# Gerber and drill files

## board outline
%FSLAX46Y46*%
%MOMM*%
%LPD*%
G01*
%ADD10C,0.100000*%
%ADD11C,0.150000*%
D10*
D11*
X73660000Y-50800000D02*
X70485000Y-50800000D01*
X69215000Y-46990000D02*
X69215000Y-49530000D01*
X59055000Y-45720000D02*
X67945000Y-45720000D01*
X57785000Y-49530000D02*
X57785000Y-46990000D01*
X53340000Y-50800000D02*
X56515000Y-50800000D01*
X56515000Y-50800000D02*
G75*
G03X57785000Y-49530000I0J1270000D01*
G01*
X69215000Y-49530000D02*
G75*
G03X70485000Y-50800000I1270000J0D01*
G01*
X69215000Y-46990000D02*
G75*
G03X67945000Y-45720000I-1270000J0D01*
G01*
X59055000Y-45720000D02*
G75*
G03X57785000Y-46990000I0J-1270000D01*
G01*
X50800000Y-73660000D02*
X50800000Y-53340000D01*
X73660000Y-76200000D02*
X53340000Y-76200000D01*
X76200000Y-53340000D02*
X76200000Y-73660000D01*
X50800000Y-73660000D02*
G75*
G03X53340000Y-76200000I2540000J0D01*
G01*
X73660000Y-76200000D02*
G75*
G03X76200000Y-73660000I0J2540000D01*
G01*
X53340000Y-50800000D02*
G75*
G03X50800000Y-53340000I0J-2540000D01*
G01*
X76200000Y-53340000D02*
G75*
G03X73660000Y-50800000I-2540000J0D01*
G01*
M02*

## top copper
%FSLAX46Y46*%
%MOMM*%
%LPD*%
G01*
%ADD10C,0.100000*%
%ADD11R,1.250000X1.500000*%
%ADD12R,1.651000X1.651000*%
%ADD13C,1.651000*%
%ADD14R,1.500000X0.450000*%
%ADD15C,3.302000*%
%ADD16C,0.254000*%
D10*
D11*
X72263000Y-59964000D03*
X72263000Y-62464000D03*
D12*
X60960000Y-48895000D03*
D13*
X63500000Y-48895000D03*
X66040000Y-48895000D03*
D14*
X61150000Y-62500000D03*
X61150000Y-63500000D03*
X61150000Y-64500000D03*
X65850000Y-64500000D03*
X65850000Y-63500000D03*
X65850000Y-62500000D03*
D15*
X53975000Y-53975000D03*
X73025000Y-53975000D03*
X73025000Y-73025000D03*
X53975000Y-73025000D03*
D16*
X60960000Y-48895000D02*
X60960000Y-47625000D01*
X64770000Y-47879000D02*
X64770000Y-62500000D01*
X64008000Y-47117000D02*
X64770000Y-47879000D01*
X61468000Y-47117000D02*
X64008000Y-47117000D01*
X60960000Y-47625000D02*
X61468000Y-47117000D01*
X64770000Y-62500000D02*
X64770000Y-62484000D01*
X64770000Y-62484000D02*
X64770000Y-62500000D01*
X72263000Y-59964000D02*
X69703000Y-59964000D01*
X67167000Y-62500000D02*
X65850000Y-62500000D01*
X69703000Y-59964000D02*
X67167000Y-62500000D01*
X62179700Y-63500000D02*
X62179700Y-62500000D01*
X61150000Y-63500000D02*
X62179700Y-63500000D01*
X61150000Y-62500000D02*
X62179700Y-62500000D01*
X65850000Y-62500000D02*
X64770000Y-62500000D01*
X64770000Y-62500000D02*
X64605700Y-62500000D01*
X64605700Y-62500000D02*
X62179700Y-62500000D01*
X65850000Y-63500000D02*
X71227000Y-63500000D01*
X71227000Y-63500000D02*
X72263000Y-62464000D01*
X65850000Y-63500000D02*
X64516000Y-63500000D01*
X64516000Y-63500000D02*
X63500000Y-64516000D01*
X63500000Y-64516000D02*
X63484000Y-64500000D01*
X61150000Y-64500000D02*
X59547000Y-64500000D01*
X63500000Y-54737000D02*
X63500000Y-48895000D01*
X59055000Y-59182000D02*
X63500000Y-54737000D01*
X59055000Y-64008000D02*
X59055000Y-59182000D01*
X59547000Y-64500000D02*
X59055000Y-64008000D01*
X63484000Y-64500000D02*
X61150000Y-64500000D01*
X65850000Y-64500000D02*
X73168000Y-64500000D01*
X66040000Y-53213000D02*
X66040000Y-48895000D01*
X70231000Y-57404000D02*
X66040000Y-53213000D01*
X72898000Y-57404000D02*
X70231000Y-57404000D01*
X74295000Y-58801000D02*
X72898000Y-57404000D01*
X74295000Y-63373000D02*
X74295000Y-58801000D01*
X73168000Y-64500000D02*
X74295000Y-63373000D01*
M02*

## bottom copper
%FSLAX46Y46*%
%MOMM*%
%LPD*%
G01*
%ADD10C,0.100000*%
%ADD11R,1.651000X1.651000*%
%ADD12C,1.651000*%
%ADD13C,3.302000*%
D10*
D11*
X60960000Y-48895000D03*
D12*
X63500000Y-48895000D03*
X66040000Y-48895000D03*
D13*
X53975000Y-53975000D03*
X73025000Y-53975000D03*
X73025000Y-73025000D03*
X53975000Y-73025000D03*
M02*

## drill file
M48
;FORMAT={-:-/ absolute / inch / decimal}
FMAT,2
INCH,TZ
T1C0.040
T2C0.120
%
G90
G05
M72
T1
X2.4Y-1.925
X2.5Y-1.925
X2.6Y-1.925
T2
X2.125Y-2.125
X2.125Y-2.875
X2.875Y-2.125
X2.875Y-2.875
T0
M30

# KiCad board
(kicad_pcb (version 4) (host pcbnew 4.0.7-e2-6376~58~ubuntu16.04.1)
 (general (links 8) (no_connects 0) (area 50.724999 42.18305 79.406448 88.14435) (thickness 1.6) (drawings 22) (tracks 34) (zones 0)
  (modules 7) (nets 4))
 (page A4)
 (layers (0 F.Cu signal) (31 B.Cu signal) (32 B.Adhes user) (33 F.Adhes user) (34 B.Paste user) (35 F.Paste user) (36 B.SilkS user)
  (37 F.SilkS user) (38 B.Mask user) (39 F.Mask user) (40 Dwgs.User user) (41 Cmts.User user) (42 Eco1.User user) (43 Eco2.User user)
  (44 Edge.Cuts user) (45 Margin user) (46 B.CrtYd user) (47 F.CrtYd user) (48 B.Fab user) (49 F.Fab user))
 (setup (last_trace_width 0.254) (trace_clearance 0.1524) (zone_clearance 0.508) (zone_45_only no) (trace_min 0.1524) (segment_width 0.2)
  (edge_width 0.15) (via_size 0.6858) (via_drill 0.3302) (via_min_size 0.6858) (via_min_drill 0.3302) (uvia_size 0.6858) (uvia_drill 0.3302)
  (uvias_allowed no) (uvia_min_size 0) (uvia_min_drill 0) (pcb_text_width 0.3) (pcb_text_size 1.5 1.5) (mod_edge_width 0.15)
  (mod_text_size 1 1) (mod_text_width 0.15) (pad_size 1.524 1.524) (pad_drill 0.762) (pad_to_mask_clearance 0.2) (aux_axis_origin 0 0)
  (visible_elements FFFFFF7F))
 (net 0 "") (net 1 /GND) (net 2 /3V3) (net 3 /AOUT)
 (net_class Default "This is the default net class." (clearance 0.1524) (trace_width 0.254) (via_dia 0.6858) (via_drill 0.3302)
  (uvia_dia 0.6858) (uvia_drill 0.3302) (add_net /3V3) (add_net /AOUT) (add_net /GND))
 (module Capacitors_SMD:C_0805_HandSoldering (layer F.Cu) (at 72.263 61.214 270)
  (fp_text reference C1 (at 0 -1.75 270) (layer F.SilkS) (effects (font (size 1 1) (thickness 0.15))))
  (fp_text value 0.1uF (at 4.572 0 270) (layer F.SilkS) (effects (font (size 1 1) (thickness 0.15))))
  (pad 1 smd rect (at -1.25 0 270) (size 1.5 1.25) (layers F.Cu F.Paste F.Mask) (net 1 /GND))
  (pad 2 smd rect (at 1.25 0 270) (size 1.5 1.25) (layers F.Cu F.Paste F.Mask) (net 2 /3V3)))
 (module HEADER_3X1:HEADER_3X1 (layer F.Cu) (at 63.5 48.895)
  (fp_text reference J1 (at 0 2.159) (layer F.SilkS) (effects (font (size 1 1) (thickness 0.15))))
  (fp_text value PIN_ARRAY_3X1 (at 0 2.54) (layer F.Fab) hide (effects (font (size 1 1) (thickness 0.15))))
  (pad 1 thru_hole rect (at -2.54 0) (size 1.651 1.651) (drill 1.016) (layers *.Cu *.Mask) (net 1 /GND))
  (pad 2 thru_hole circle (at 0 0) (size 1.651 1.651) (drill 1.016) (layers *.Cu *.Mask) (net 2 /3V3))
  (pad 3 thru_hole circle (at 2.54 0) (size 1.651 1.651) (drill 1.016) (layers *.Cu *.Mask) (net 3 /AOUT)))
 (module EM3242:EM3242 (layer F.Cu) (at 63.5 63.5)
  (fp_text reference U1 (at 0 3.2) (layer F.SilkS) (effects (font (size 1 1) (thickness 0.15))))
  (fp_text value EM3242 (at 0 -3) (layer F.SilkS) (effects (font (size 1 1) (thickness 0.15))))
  (pad 1 smd rect (at -2.35 -1) (size 1.5 0.45) (layers F.Cu F.Paste F.Mask) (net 1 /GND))
  (pad 2 smd rect (at -2.35 0) (size 1.5 0.45) (layers F.Cu F.Paste F.Mask) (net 1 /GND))
  (pad 3 smd rect (at -2.35 1) (size 1.5 0.45) (layers F.Cu F.Paste F.Mask) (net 2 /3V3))
  (pad 4 smd rect (at 2.35 1) (size 1.5 0.45) (layers F.Cu F.Paste F.Mask) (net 3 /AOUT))
  (pad 5 smd rect (at 2.35 0) (size 1.5 0.45) (layers F.Cu F.Paste F.Mask) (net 2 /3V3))
  (pad 6 smd rect (at 2.35 -1) (size 1.5 0.45) (layers F.Cu F.Paste F.Mask) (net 1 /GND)))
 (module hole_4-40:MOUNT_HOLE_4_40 (layer F.Cu) (at 53.34 53.34)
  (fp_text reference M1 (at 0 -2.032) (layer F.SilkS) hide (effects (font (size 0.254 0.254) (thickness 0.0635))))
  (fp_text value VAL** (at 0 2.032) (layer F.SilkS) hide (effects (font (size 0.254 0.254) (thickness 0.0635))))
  (pad "" thru_hole circle (at 0.635 0.635) (size 3.302 3.302) (drill 3.048) (layers *.Cu *.SilkS *.Mask)))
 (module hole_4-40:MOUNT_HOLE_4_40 (layer F.Cu) (at 75.057 44.577)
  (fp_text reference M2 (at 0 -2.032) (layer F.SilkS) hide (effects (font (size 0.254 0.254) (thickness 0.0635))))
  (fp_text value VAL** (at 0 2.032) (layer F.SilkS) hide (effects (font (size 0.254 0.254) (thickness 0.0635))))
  (pad "" thru_hole circle (at -2.032 9.398) (size 3.302 3.302) (drill 3.048) (layers *.Cu *.SilkS *.Mask)))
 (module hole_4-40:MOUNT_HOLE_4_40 (layer F.Cu) (at 78.74 85.725)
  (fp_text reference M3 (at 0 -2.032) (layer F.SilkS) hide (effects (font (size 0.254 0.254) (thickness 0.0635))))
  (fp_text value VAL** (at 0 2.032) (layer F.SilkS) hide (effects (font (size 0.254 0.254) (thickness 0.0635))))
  (pad "" thru_hole circle (at -5.715 -12.7) (size 3.302 3.302) (drill 3.048) (layers *.Cu *.SilkS *.Mask)))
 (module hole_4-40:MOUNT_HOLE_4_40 (layer F.Cu) (at 52.324 85.09)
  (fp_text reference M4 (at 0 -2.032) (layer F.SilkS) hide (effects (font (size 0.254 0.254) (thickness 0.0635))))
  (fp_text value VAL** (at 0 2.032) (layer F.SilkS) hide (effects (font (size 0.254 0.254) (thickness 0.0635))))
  (pad "" thru_hole circle (at 1.651 -12.065) (size 3.302 3.302) (drill 3.048) (layers *.Cu *.SilkS *.Mask)))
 (gr_line (start 73.66 50.8) (end 70.485 50.8) (angle 90) (layer Edge.Cuts) (width 0.15))
 (gr_line (start 69.215 46.99) (end 69.215 49.53) (angle 90) (layer Edge.Cuts) (width 0.15))
 (gr_line (start 59.055 45.72) (end 67.945 45.72) (angle 90) (layer Edge.Cuts) (width 0.15))
 (gr_line (start 57.785 49.53) (end 57.785 46.99) (angle 90) (layer Edge.Cuts) (width 0.15))
 (gr_line (start 53.34 50.8) (end 56.515 50.8) (angle 90) (layer Edge.Cuts) (width 0.15))
 (gr_arc (start 56.515 49.53) (end 57.785 49.53) (angle 90) (layer Edge.Cuts) (width 0.15))
 (gr_arc (start 70.485 49.53) (end 70.485 50.8) (angle 90) (layer Edge.Cuts) (width 0.15))
 (gr_arc (start 67.945 46.99) (end 67.945 45.72) (angle 90) (layer Edge.Cuts) (width 0.15))
 (gr_arc (start 59.055 46.99) (end 57.785 46.99) (angle 90) (layer Edge.Cuts) (width 0.15))
 (gr_line (start 50.8 73.66) (end 50.8 53.34) (angle 90) (layer Edge.Cuts) (width 0.15))
 (gr_line (start 73.66 76.2) (end 53.34 76.2) (angle 90) (layer Edge.Cuts) (width 0.15))
 (gr_line (start 76.2 53.34) (end 76.2 73.66) (angle 90) (layer Edge.Cuts) (width 0.15))
 (gr_arc (start 53.34 73.66) (end 53.34 76.2) (angle 90) (layer Edge.Cuts) (width 0.15))
 (gr_arc (start 73.66 73.66) (end 76.2 73.66) (angle 90) (layer Edge.Cuts) (width 0.15))
 (gr_arc (start 53.34 53.34) (end 50.8 53.34) (angle 90) (layer Edge.Cuts) (width 0.15))
 (gr_arc (start 73.66 53.34) (end 73.66 50.8) (angle 90) (layer Edge.Cuts) (width 0.15))
 (segment (start 60.96 48.895) (end 60.96 47.625) (width 0.254) (layer F.Cu) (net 1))
 (segment (start 64.77 47.879) (end 64.77 62.5) (width 0.254) (layer F.Cu) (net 1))
 (segment (start 64.008 47.117) (end 64.77 47.879) (width 0.254) (layer F.Cu) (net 1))
 (segment (start 61.468 47.117) (end 64.008 47.117) (width 0.254) (layer F.Cu) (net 1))
 (segment (start 60.96 47.625) (end 61.468 47.117) (width 0.254) (layer F.Cu) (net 1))
 (segment (start 64.77 62.5) (end 64.77 62.484) (width 0.254) (layer F.Cu) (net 1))
 (segment (start 64.77 62.484) (end 64.77 62.5) (width 0.254) (layer F.Cu) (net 1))
 (segment (start 72.263 59.964) (end 69.703 59.964) (width 0.254) (layer F.Cu) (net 1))
 (segment (start 67.167 62.5) (end 65.85 62.5) (width 0.254) (layer F.Cu) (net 1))
 (segment (start 69.703 59.964) (end 67.167 62.5) (width 0.254) (layer F.Cu) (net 1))
 (segment (start 62.1797 63.5) (end 62.1797 62.5) (width 0.254) (layer F.Cu) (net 1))
 (segment (start 61.15 63.5) (end 62.1797 63.5) (width 0.254) (layer F.Cu) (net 1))
 (segment (start 61.15 62.5) (end 62.1797 62.5) (width 0.254) (layer F.Cu) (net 1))
 (segment (start 65.85 62.5) (end 64.77 62.5) (width 0.254) (layer F.Cu) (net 1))
 (segment (start 64.77 62.5) (end 64.6057 62.5) (width 0.254) (layer F.Cu) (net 1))
 (segment (start 64.6057 62.5) (end 62.1797 62.5) (width 0.254) (layer F.Cu) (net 1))
 (segment (start 65.85 63.5) (end 71.227 63.5) (width 0.254) (layer F.Cu) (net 2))
 (segment (start 71.227 63.5) (end 72.263 62.464) (width 0.254) (layer F.Cu) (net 2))
 (segment (start 65.85 63.5) (end 64.516 63.5) (width 0.254) (layer F.Cu) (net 2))
 (segment (start 64.516 63.5) (end 63.5 64.516) (width 0.254) (layer F.Cu) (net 2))
 (segment (start 63.5 64.516) (end 63.484 64.5) (width 0.254) (layer F.Cu) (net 2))
 (segment (start 61.15 64.5) (end 59.547 64.5) (width 0.254) (layer F.Cu) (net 2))
 (segment (start 63.5 54.737) (end 63.5 48.895) (width 0.254) (layer F.Cu) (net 2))
 (segment (start 59.055 59.182) (end 63.5 54.737) (width 0.254) (layer F.Cu) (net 2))
 (segment (start 59.055 64.008) (end 59.055 59.182) (width 0.254) (layer F.Cu) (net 2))
 (segment (start 59.547 64.5) (end 59.055 64.008) (width 0.254) (layer F.Cu) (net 2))
 (segment (start 63.484 64.5) (end 61.15 64.5) (width 0.254) (layer F.Cu) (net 2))
 (segment (start 65.85 64.5) (end 73.168 64.5) (width 0.254) (layer F.Cu) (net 3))
 (segment (start 66.04 53.213) (end 66.04 48.895) (width 0.254) (layer F.Cu) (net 3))
 (segment (start 70.231 57.404) (end 66.04 53.213) (width 0.254) (layer F.Cu) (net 3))
 (segment (start 72.898 57.404) (end 70.231 57.404) (width 0.254) (layer F.Cu) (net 3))
 (segment (start 74.295 58.801) (end 72.898 57.404) (width 0.254) (layer F.Cu) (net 3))
 (segment (start 74.295 63.373) (end 74.295 58.801) (width 0.254) (layer F.Cu) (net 3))
 (segment (start 73.168 64.5) (end 74.295 63.373) (width 0.254) (layer F.Cu) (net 3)))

